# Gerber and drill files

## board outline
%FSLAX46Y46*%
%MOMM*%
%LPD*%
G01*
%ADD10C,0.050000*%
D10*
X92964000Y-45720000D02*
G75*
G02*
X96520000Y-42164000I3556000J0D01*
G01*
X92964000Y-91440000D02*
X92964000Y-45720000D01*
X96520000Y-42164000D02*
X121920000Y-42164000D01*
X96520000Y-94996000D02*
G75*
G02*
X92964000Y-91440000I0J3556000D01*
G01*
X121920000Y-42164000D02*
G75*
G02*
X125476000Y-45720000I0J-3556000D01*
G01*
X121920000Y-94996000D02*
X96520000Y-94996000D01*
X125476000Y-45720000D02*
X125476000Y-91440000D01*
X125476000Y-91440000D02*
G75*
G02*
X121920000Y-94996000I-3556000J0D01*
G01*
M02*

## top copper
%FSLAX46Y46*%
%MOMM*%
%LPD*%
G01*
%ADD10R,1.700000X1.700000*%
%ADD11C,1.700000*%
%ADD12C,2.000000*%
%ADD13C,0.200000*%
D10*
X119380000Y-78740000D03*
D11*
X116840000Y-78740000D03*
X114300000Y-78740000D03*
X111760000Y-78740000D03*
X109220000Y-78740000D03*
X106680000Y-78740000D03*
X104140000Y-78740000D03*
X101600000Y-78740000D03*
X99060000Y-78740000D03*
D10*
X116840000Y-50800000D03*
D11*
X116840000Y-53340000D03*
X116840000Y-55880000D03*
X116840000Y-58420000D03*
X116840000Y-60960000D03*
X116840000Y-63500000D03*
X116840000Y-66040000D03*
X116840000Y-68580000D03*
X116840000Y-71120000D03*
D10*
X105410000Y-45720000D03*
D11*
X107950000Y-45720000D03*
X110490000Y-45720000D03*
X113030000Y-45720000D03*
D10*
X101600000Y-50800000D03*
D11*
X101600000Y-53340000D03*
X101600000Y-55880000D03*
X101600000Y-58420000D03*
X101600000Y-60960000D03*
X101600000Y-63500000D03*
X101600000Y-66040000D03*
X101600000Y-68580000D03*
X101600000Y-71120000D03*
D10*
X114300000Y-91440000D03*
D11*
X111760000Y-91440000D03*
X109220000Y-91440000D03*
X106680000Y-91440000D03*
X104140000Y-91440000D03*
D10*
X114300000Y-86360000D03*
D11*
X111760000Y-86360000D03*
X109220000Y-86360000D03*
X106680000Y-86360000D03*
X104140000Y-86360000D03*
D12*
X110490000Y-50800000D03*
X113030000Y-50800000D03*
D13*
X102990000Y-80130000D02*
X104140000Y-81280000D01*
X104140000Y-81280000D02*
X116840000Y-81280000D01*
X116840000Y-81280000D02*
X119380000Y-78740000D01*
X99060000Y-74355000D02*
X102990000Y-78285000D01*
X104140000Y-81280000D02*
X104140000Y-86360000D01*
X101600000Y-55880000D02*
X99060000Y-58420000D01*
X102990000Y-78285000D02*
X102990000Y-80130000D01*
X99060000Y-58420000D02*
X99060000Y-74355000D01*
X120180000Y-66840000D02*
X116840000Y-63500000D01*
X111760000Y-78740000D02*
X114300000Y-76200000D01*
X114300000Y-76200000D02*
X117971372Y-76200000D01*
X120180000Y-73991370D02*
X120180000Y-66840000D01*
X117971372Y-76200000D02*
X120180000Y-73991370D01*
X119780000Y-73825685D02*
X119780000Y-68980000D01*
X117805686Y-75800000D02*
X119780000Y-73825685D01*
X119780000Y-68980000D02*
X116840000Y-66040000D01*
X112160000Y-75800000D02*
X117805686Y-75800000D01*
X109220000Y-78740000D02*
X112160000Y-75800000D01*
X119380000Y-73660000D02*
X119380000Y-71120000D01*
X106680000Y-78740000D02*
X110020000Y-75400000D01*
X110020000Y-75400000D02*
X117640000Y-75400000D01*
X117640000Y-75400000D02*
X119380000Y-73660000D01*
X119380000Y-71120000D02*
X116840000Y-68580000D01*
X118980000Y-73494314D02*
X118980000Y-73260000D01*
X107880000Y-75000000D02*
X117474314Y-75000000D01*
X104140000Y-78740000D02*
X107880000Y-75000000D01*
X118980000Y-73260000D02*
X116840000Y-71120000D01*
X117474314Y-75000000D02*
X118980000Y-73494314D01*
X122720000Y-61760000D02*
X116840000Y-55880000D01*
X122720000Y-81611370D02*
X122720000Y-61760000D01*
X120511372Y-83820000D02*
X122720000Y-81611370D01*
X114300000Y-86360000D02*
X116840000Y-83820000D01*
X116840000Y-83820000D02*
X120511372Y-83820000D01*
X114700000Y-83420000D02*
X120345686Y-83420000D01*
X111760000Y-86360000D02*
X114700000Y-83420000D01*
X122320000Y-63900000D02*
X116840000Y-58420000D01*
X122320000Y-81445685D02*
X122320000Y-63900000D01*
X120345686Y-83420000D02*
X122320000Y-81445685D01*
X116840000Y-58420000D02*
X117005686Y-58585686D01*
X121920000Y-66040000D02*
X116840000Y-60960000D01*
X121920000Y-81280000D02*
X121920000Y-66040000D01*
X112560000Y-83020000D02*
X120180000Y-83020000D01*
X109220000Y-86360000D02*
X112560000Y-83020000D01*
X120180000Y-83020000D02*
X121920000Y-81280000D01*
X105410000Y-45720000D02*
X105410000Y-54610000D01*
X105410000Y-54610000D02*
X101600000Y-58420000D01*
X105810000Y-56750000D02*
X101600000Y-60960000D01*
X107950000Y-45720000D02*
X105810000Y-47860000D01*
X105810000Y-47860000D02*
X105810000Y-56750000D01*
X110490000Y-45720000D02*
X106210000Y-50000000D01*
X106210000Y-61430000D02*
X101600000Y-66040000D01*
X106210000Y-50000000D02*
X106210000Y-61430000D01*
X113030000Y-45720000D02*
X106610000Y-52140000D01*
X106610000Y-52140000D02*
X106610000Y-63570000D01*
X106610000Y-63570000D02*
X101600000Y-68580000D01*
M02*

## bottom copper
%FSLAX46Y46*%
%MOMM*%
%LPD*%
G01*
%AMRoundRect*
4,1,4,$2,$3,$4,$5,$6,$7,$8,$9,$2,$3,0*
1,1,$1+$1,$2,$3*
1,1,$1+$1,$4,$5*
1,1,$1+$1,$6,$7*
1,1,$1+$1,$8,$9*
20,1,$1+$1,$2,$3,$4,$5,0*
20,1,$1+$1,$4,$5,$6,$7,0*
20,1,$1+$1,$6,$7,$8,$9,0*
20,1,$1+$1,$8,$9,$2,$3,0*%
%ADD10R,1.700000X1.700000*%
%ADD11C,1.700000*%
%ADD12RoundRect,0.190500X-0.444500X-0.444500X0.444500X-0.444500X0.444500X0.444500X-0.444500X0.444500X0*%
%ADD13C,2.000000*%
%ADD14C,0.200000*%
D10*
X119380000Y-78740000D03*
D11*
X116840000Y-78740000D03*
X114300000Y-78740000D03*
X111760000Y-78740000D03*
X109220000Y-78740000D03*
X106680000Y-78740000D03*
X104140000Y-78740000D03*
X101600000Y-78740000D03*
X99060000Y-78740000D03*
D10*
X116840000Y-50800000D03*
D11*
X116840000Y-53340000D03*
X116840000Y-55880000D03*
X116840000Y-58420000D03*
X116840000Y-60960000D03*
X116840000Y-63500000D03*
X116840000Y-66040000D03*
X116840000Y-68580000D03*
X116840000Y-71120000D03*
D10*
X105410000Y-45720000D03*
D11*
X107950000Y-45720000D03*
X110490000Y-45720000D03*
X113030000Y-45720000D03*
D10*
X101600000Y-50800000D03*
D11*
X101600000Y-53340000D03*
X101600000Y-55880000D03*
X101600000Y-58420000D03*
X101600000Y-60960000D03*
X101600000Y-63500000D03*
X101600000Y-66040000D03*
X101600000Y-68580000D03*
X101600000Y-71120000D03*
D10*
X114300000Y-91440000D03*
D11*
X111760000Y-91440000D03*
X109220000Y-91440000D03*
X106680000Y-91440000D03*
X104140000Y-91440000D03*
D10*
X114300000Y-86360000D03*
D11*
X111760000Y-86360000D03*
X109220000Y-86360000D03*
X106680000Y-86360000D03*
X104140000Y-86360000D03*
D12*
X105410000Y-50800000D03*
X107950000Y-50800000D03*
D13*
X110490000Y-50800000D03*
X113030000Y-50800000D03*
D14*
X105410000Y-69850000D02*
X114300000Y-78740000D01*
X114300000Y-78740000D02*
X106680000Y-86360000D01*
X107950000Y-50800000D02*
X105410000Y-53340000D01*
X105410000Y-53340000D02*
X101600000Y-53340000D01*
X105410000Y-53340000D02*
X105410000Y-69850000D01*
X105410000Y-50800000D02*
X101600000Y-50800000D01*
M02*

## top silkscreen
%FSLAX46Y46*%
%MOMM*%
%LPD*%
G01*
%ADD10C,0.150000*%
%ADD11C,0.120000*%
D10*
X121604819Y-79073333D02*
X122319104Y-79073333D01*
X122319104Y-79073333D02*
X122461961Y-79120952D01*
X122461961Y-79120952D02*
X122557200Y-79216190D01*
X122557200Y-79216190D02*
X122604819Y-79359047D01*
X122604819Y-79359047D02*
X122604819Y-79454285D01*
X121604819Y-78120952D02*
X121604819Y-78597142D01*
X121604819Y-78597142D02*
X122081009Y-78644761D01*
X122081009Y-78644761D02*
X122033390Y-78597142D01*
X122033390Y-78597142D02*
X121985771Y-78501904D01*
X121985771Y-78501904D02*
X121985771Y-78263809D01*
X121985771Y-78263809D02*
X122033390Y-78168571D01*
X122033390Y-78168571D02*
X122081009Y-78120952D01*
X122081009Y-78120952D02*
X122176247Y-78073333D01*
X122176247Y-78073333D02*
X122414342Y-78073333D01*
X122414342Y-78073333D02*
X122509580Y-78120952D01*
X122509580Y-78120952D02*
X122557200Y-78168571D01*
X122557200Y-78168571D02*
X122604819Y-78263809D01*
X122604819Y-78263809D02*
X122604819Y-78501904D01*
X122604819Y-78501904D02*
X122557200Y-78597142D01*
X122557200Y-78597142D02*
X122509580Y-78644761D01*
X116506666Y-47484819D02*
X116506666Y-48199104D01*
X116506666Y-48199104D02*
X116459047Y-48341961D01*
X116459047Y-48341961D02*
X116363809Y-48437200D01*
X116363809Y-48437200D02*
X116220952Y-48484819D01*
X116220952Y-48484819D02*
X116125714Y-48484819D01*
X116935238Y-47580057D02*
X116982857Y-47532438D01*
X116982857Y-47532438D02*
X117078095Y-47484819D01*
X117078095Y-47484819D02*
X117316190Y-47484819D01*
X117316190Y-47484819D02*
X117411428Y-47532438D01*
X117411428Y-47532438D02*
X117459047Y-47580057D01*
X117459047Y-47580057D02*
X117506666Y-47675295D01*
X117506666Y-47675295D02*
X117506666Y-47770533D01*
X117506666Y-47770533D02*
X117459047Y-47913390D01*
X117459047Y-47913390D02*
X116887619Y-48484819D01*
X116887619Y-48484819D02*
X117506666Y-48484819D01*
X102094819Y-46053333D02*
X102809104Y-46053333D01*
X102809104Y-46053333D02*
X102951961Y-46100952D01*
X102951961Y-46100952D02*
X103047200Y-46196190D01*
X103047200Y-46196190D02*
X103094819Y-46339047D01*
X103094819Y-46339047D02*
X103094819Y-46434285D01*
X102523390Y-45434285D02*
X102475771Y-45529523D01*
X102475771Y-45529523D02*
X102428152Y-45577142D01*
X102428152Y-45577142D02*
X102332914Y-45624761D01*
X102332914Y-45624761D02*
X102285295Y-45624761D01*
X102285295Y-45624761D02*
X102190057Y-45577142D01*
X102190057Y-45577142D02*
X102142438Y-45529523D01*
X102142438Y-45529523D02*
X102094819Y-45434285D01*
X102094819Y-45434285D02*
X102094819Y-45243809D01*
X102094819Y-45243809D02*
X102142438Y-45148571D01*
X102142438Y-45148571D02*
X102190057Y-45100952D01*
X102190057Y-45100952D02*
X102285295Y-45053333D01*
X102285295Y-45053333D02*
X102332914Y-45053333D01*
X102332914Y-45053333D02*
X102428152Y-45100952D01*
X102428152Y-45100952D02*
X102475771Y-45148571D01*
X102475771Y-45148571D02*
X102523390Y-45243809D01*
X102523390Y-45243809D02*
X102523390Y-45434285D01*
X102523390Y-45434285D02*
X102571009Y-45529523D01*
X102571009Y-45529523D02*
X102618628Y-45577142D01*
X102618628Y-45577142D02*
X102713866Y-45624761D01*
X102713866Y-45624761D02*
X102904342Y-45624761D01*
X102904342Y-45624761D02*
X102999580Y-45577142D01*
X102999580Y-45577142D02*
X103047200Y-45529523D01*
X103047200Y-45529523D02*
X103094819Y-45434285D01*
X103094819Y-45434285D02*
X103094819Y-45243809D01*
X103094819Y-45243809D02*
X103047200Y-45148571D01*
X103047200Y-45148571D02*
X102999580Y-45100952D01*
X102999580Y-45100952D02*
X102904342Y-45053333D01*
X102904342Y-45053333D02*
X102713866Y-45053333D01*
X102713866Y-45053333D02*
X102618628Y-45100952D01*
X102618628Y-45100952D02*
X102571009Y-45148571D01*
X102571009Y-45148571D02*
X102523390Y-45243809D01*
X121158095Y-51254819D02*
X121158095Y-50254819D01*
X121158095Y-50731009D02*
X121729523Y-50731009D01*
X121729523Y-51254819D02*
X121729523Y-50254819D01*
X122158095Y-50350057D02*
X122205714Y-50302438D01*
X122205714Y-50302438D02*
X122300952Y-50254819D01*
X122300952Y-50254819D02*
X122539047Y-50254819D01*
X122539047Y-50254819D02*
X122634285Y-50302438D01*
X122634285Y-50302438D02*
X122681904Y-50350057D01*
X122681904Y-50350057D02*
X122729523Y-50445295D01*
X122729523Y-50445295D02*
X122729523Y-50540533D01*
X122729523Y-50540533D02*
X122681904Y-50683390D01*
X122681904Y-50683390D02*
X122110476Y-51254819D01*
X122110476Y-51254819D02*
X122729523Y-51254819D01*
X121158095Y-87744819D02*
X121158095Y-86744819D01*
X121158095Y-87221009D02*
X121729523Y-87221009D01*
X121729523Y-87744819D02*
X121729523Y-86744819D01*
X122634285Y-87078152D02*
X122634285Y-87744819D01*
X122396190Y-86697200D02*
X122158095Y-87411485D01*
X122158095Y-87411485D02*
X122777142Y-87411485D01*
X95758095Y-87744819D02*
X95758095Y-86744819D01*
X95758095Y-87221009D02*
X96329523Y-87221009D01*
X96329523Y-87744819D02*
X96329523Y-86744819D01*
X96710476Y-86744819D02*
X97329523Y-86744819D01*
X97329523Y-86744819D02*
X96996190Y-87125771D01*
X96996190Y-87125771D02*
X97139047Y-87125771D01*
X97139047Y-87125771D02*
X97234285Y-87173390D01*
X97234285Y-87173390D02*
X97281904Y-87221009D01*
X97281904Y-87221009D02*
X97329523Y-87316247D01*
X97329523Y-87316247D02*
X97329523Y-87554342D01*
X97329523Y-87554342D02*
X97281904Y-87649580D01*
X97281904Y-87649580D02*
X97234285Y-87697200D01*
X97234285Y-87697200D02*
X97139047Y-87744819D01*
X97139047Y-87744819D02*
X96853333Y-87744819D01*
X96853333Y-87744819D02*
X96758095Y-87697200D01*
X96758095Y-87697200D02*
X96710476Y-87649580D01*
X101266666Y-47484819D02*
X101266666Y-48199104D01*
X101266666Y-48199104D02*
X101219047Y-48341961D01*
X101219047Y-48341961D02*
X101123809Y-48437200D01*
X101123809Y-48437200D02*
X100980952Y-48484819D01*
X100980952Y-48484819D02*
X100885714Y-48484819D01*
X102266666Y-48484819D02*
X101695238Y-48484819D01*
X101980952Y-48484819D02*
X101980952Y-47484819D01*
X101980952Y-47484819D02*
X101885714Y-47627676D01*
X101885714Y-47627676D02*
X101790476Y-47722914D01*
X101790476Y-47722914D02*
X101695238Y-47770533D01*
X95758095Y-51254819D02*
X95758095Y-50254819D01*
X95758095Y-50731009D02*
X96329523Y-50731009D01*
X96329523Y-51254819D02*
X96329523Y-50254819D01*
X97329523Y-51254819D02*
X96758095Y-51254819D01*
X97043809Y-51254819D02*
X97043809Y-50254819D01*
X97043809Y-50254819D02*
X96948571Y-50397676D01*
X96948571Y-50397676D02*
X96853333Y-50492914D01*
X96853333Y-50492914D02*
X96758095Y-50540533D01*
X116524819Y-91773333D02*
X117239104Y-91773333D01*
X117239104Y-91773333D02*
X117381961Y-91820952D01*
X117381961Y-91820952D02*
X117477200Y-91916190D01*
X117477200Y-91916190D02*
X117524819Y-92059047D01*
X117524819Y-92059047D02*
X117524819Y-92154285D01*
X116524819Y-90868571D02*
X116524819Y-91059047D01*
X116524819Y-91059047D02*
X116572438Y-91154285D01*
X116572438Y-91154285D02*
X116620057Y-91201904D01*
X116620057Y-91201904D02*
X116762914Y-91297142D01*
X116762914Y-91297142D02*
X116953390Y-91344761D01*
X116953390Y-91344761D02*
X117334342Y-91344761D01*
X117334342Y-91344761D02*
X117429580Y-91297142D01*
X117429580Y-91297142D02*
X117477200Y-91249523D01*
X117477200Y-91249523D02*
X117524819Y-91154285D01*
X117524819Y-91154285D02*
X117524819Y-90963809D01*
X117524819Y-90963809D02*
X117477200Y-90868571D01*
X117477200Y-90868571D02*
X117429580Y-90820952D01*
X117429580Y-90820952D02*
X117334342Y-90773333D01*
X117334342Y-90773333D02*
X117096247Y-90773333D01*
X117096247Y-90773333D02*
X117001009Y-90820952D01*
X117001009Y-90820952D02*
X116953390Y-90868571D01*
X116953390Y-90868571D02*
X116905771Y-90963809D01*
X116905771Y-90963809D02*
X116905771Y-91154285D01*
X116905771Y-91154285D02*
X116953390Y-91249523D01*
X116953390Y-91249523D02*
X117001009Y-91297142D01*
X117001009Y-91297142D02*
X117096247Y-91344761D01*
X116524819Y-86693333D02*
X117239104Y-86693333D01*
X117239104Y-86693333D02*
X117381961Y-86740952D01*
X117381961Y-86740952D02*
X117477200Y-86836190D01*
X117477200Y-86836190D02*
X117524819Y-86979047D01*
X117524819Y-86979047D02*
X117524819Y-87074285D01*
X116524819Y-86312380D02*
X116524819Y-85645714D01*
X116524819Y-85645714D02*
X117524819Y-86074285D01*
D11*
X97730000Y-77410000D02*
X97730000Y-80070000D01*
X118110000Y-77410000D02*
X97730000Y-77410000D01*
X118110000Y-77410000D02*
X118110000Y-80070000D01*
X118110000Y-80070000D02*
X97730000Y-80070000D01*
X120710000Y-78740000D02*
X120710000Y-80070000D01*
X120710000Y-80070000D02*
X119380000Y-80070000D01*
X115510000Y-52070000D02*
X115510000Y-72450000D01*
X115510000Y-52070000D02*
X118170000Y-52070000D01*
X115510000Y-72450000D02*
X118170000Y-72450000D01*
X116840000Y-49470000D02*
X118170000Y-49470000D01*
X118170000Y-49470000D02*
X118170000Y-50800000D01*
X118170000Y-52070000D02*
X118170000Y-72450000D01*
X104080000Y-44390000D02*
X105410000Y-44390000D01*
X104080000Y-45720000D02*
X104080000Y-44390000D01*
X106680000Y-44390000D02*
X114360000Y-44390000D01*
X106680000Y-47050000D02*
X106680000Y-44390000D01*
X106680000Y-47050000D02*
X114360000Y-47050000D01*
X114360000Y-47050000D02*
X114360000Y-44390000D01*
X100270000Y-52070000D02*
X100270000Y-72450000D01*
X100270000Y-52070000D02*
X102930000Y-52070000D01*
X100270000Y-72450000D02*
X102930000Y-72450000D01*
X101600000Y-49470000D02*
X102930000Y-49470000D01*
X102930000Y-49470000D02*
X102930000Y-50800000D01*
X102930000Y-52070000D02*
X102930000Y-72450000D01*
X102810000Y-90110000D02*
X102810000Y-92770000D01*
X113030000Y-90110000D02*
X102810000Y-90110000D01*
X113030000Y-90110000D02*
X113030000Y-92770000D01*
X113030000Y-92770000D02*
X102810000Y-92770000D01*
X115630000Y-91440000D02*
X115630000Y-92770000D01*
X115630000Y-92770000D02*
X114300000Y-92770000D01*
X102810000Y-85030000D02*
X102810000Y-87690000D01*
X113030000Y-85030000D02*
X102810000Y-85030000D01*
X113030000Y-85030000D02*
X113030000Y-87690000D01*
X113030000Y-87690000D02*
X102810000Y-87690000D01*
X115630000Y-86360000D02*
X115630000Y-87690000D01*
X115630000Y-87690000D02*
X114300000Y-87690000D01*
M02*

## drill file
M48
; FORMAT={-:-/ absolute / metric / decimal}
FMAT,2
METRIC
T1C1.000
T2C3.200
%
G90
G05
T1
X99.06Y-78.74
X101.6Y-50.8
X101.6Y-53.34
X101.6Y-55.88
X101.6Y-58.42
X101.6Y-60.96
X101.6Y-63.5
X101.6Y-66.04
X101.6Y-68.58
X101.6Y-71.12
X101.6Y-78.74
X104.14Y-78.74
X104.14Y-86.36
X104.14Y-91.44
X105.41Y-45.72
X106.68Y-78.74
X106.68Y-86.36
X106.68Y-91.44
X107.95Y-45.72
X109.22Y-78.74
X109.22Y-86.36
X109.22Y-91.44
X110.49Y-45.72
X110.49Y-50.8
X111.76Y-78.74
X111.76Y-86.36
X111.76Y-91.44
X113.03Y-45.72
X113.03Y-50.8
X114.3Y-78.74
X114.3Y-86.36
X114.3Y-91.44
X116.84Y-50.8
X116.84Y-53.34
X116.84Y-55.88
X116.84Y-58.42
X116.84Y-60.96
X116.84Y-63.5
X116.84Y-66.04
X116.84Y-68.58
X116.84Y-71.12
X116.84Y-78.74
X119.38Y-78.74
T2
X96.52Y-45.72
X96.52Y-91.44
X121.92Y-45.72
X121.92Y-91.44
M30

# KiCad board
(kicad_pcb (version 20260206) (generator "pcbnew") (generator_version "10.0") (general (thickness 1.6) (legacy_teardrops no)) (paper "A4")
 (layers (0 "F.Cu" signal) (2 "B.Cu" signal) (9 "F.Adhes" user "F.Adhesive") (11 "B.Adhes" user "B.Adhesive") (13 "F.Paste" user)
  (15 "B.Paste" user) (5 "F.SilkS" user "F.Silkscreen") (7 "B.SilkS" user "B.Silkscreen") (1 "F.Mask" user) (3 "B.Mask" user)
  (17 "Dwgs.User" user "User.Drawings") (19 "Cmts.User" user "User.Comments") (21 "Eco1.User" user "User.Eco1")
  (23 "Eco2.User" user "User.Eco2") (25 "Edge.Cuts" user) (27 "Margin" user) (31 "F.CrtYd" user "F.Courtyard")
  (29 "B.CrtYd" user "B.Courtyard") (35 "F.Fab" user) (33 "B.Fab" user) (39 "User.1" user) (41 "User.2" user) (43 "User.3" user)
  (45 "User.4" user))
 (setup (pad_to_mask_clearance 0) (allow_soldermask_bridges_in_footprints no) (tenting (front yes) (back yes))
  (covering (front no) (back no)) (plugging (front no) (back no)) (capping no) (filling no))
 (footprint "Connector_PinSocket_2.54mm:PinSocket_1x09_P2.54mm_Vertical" (layer "F.Cu") (at 119.38 78.74 -90)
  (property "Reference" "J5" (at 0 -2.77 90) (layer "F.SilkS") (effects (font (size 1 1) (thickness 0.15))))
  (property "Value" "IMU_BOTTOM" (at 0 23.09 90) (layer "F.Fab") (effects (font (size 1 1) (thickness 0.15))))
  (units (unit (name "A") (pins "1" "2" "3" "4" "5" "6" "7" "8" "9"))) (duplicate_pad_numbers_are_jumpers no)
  (fp_line (start -1.33 21.65) (end 1.33 21.65) (stroke (width 0.12) (type solid)) (layer "F.SilkS"))
  (fp_line (start -1.33 1.27) (end -1.33 21.65) (stroke (width 0.12) (type solid)) (layer "F.SilkS"))
  (fp_line (start -1.33 1.27) (end 1.33 1.27) (stroke (width 0.12) (type solid)) (layer "F.SilkS"))
  (fp_line (start 1.33 1.27) (end 1.33 21.65) (stroke (width 0.12) (type solid)) (layer "F.SilkS"))
  (fp_line (start 0 -1.33) (end 1.33 -1.33) (stroke (width 0.12) (type solid)) (layer "F.SilkS"))
  (fp_line (start 1.33 -1.33) (end 1.33 0) (stroke (width 0.12) (type solid)) (layer "F.SilkS"))
  (pad "1" thru_hole rect (at 0 0 270) (size 1.7 1.7) (drill 1) (layers "*.Cu" "*.Mask") (remove_unused_layers no) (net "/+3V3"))
  (pad "2" thru_hole circle (at 0 2.54 270) (size 1.7 1.7) (drill 1) (layers "*.Cu" "*.Mask") (remove_unused_layers no)
   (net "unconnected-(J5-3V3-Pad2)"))
  (pad "3" thru_hole circle (at 0 5.08 270) (size 1.7 1.7) (drill 1) (layers "*.Cu" "*.Mask") (remove_unused_layers no) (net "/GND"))
  (pad "4" thru_hole circle (at 0 7.62 270) (size 1.7 1.7) (drill 1) (layers "*.Cu" "*.Mask") (remove_unused_layers no) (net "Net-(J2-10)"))
  (pad "5" thru_hole circle (at 0 10.16 270) (size 1.7 1.7) (drill 1) (layers "*.Cu" "*.Mask") (remove_unused_layers no) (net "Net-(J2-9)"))
  (pad "6" thru_hole circle (at 0 12.7 270) (size 1.7 1.7) (drill 1) (layers "*.Cu" "*.Mask") (remove_unused_layers no) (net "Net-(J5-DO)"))
  (pad "7" thru_hole circle (at 0 15.24 270) (size 1.7 1.7) (drill 1) (layers "*.Cu" "*.Mask") (remove_unused_layers no) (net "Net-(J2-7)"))
  (pad "8" thru_hole circle (at 0 17.78 270) (size 1.7 1.7) (drill 1) (layers "*.Cu" "*.Mask") (remove_unused_layers no)
   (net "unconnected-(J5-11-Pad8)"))
  (pad "9" thru_hole circle (at 0 20.32 270) (size 1.7 1.7) (drill 1) (layers "*.Cu" "*.Mask") (remove_unused_layers no)
   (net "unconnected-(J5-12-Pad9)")))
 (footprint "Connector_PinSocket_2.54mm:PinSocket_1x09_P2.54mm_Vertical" (layer "F.Cu") (at 116.84 50.8)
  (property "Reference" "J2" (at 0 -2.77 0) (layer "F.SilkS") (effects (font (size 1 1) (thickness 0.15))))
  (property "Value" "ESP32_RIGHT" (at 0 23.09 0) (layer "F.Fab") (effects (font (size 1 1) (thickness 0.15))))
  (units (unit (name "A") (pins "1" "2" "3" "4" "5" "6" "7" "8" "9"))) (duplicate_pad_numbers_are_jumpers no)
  (fp_line (start -1.33 1.27) (end -1.33 21.65) (stroke (width 0.12) (type solid)) (layer "F.SilkS"))
  (fp_line (start -1.33 1.27) (end 1.33 1.27) (stroke (width 0.12) (type solid)) (layer "F.SilkS"))
  (fp_line (start -1.33 21.65) (end 1.33 21.65) (stroke (width 0.12) (type solid)) (layer "F.SilkS"))
  (fp_line (start 0 -1.33) (end 1.33 -1.33) (stroke (width 0.12) (type solid)) (layer "F.SilkS"))
  (fp_line (start 1.33 -1.33) (end 1.33 0) (stroke (width 0.12) (type solid)) (layer "F.SilkS"))
  (fp_line (start 1.33 1.27) (end 1.33 21.65) (stroke (width 0.12) (type solid)) (layer "F.SilkS"))
  (pad "1" thru_hole rect (at 0 0) (size 1.7 1.7) (drill 1) (layers "*.Cu" "*.Mask") (remove_unused_layers no)
   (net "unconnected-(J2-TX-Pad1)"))
  (pad "2" thru_hole circle (at 0 2.54) (size 1.7 1.7) (drill 1) (layers "*.Cu" "*.Mask") (remove_unused_layers no)
   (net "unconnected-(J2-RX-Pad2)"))
  (pad "3" thru_hole circle (at 0 5.08) (size 1.7 1.7) (drill 1) (layers "*.Cu" "*.Mask") (remove_unused_layers no) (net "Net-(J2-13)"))
  (pad "4" thru_hole circle (at 0 7.62) (size 1.7 1.7) (drill 1) (layers "*.Cu" "*.Mask") (remove_unused_layers no) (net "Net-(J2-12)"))
  (pad "5" thru_hole circle (at 0 10.16) (size 1.7 1.7) (drill 1) (layers "*.Cu" "*.Mask") (remove_unused_layers no) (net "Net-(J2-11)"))
  (pad "6" thru_hole circle (at 0 12.7) (size 1.7 1.7) (drill 1) (layers "*.Cu" "*.Mask") (remove_unused_layers no) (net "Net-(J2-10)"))
  (pad "7" thru_hole circle (at 0 15.24) (size 1.7 1.7) (drill 1) (layers "*.Cu" "*.Mask") (remove_unused_layers no) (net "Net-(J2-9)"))
  (pad "8" thru_hole circle (at 0 17.78) (size 1.7 1.7) (drill 1) (layers "*.Cu" "*.Mask") (remove_unused_layers no) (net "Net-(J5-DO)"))
  (pad "9" thru_hole circle (at 0 20.32) (size 1.7 1.7) (drill 1) (layers "*.Cu" "*.Mask") (remove_unused_layers no) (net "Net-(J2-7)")))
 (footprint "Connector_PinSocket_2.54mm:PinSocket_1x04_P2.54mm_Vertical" (layer "F.Cu") (at 105.41 45.72 90)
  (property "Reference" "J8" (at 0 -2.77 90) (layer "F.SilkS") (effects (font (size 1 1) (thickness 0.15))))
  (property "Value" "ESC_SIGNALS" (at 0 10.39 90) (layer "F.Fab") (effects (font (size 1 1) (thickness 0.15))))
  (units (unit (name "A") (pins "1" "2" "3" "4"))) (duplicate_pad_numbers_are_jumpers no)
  (fp_line (start 1.33 -1.33) (end 1.33 0) (stroke (width 0.12) (type solid)) (layer "F.SilkS"))
  (fp_line (start 0 -1.33) (end 1.33 -1.33) (stroke (width 0.12) (type solid)) (layer "F.SilkS"))
  (fp_line (start 1.33 1.27) (end 1.33 8.95) (stroke (width 0.12) (type solid)) (layer "F.SilkS"))
  (fp_line (start -1.33 1.27) (end 1.33 1.27) (stroke (width 0.12) (type solid)) (layer "F.SilkS"))
  (fp_line (start -1.33 1.27) (end -1.33 8.95) (stroke (width 0.12) (type solid)) (layer "F.SilkS"))
  (fp_line (start -1.33 8.95) (end 1.33 8.95) (stroke (width 0.12) (type solid)) (layer "F.SilkS"))
  (pad "1" thru_hole rect (at 0 0 90) (size 1.7 1.7) (drill 1) (layers "*.Cu" "*.Mask") (remove_unused_layers no) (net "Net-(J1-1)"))
  (pad "2" thru_hole circle (at 0 2.54 90) (size 1.7 1.7) (drill 1) (layers "*.Cu" "*.Mask") (remove_unused_layers no) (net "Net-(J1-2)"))
  (pad "3" thru_hole circle (at 0 5.08 90) (size 1.7 1.7) (drill 1) (layers "*.Cu" "*.Mask") (remove_unused_layers no) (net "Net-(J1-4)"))
  (pad "4" thru_hole circle (at 0 7.62 90) (size 1.7 1.7) (drill 1) (layers "*.Cu" "*.Mask") (remove_unused_layers no) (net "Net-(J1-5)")))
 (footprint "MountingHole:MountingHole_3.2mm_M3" (layer "F.Cu") (at 121.92 45.72)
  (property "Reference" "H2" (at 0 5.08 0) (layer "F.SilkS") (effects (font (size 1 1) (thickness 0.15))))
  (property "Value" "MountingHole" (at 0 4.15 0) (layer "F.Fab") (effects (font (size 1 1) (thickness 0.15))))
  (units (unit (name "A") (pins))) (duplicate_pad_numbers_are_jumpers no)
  (pad "" np_thru_hole circle (at 0 0) (size 3.2 3.2) (drill 3.2) (layers "*.Cu" "*.Mask")))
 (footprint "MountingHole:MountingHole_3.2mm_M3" (layer "F.Cu") (at 121.92 91.44)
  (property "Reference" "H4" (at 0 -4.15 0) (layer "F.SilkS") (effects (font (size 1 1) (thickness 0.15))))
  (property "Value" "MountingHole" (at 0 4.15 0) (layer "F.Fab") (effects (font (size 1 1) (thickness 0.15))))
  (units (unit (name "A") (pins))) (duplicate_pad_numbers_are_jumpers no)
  (pad "" np_thru_hole circle (at 0 0) (size 3.2 3.2) (drill 3.2) (layers "*.Cu" "*.Mask")))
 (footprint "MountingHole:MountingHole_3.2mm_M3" (layer "F.Cu") (at 96.52 91.44)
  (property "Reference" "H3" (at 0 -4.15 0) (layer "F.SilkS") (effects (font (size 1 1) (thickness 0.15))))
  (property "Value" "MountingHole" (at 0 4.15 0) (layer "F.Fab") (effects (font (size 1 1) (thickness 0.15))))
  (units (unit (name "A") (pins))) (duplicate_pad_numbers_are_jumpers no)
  (pad "" np_thru_hole circle (at 0 0) (size 3.2 3.2) (drill 3.2) (layers "*.Cu" "*.Mask")))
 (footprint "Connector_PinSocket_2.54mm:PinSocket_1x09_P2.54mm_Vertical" (layer "F.Cu") (at 101.6 50.8)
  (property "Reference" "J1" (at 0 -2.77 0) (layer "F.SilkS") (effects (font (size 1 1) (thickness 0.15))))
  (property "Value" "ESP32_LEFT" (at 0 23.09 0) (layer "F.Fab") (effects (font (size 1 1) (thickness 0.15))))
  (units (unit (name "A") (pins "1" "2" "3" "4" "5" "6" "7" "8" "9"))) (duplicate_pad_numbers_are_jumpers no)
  (fp_line (start -1.33 1.27) (end -1.33 21.65) (stroke (width 0.12) (type solid)) (layer "F.SilkS"))
  (fp_line (start -1.33 1.27) (end 1.33 1.27) (stroke (width 0.12) (type solid)) (layer "F.SilkS"))
  (fp_line (start -1.33 21.65) (end 1.33 21.65) (stroke (width 0.12) (type solid)) (layer "F.SilkS"))
  (fp_line (start 0 -1.33) (end 1.33 -1.33) (stroke (width 0.12) (type solid)) (layer "F.SilkS"))
  (fp_line (start 1.33 -1.33) (end 1.33 0) (stroke (width 0.12) (type solid)) (layer "F.SilkS"))
  (fp_line (start 1.33 1.27) (end 1.33 21.65) (stroke (width 0.12) (type solid)) (layer "F.SilkS"))
  (pad "1" thru_hole rect (at 0 0) (size 1.7 1.7) (drill 1) (layers "*.Cu" "*.Mask") (remove_unused_layers no) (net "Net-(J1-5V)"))
  (pad "2" thru_hole circle (at 0 2.54) (size 1.7 1.7) (drill 1) (layers "*.Cu" "*.Mask") (remove_unused_layers no) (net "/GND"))
  (pad "3" thru_hole circle (at 0 5.08) (size 1.7 1.7) (drill 1) (layers "*.Cu" "*.Mask") (remove_unused_layers no) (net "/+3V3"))
  (pad "4" thru_hole circle (at 0 7.62) (size 1.7 1.7) (drill 1) (layers "*.Cu" "*.Mask") (remove_unused_layers no) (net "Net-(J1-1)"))
  (pad "5" thru_hole circle (at 0 10.16) (size 1.7 1.7) (drill 1) (layers "*.Cu" "*.Mask") (remove_unused_layers no) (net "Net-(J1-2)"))
  (pad "6" thru_hole circle (at 0 12.7) (size 1.7 1.7) (drill 1) (layers "*.Cu" "*.Mask") (remove_unused_layers no)
   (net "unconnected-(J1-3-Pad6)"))
  (pad "7" thru_hole circle (at 0 15.24) (size 1.7 1.7) (drill 1) (layers "*.Cu" "*.Mask") (remove_unused_layers no) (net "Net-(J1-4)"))
  (pad "8" thru_hole circle (at 0 17.78) (size 1.7 1.7) (drill 1) (layers "*.Cu" "*.Mask") (remove_unused_layers no) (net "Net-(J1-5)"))
  (pad "9" thru_hole circle (at 0 20.32) (size 1.7 1.7) (drill 1) (layers "*.Cu" "*.Mask") (remove_unused_layers no)
   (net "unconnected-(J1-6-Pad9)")))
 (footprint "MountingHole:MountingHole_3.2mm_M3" (layer "F.Cu") (at 96.52 45.72)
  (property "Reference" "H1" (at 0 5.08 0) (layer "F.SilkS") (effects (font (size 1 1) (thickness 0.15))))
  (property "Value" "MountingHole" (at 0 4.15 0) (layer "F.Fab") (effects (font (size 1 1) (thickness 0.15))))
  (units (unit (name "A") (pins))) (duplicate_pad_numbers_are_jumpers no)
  (pad "" np_thru_hole circle (at 0 0) (size 3.2 3.2) (drill 3.2) (layers "*.Cu" "*.Mask")))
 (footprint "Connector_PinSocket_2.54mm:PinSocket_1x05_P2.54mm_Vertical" (layer "F.Cu") (at 114.3 91.44 -90)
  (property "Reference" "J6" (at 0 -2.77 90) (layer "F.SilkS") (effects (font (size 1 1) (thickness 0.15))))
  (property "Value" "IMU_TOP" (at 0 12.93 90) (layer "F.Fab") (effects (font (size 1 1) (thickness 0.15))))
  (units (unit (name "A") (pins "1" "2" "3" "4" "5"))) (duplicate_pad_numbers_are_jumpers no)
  (fp_line (start -1.33 11.49) (end 1.33 11.49) (stroke (width 0.12) (type solid)) (layer "F.SilkS"))
  (fp_line (start -1.33 1.27) (end -1.33 11.49) (stroke (width 0.12) (type solid)) (layer "F.SilkS"))
  (fp_line (start -1.33 1.27) (end 1.33 1.27) (stroke (width 0.12) (type solid)) (layer "F.SilkS"))
  (fp_line (start 1.33 1.27) (end 1.33 11.49) (stroke (width 0.12) (type solid)) (layer "F.SilkS"))
  (fp_line (start 0 -1.33) (end 1.33 -1.33) (stroke (width 0.12) (type solid)) (layer "F.SilkS"))
  (fp_line (start 1.33 -1.33) (end 1.33 0) (stroke (width 0.12) (type solid)) (layer "F.SilkS"))
  (pad "1" thru_hole rect (at 0 0 270) (size 1.7 1.7) (drill 1) (layers "*.Cu" "*.Mask") (remove_unused_layers no)
   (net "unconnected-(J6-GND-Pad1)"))
  (pad "2" thru_hole circle (at 0 2.54 270) (size 1.7 1.7) (drill 1) (layers "*.Cu" "*.Mask") (remove_unused_layers no)
   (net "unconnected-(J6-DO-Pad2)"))
  (pad "3" thru_hole circle (at 0 5.08 270) (size 1.7 1.7) (drill 1) (layers "*.Cu" "*.Mask") (remove_unused_layers no)
   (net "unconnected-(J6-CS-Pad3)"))
  (pad "4" thru_hole circle (at 0 7.62 270) (size 1.7 1.7) (drill 1) (layers "*.Cu" "*.Mask") (remove_unused_layers no)
   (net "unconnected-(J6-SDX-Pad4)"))
  (pad "5" thru_hole circle (at 0 10.16 270) (size 1.7 1.7) (drill 1) (layers "*.Cu" "*.Mask") (remove_unused_layers no)
   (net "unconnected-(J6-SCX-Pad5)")))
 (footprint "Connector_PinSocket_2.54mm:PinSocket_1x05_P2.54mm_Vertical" (layer "F.Cu") (at 114.3 86.36 -90)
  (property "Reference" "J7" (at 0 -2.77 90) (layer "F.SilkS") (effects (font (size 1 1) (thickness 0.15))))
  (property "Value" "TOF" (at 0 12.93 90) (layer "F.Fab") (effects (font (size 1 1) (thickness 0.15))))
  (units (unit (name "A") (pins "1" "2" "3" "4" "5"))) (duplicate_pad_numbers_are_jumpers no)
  (fp_line (start -1.33 11.49) (end 1.33 11.49) (stroke (width 0.12) (type solid)) (layer "F.SilkS"))
  (fp_line (start -1.33 1.27) (end -1.33 11.49) (stroke (width 0.12) (type solid)) (layer "F.SilkS"))
  (fp_line (start -1.33 1.27) (end 1.33 1.27) (stroke (width 0.12) (type solid)) (layer "F.SilkS"))
  (fp_line (start 1.33 1.27) (end 1.33 11.49) (stroke (width 0.12) (type solid)) (layer "F.SilkS"))
  (fp_line (start 0 -1.33) (end 1.33 -1.33) (stroke (width 0.12) (type solid)) (layer "F.SilkS"))
  (fp_line (start 1.33 -1.33) (end 1.33 0) (stroke (width 0.12) (type solid)) (layer "F.SilkS"))
  (pad "1" thru_hole rect (at 0 0 270) (size 1.7 1.7) (drill 1) (layers "*.Cu" "*.Mask") (remove_unused_layers no) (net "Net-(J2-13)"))
  (pad "2" thru_hole circle (at 0 2.54 270) (size 1.7 1.7) (drill 1) (layers "*.Cu" "*.Mask") (remove_unused_layers no) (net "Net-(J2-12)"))
  (pad "3" thru_hole circle (at 0 5.08 270) (size 1.7 1.7) (drill 1) (layers "*.Cu" "*.Mask") (remove_unused_layers no) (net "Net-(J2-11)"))
  (pad "4" thru_hole circle (at 0 7.62 270) (size 1.7 1.7) (drill 1) (layers "*.Cu" "*.Mask") (remove_unused_layers no) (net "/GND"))
  (pad "5" thru_hole circle (at 0 10.16 270) (size 1.7 1.7) (drill 1) (layers "*.Cu" "*.Mask") (remove_unused_layers no) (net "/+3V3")))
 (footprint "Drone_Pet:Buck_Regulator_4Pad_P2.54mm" (layer "B.Cu") (at 105.41 50.8)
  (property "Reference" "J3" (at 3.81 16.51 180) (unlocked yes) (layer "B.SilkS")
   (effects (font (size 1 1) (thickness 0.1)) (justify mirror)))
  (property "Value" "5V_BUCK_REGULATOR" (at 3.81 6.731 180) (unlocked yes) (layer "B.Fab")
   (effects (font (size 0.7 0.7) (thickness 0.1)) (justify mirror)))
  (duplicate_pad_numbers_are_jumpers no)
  (pad "1" smd roundrect (at 0 0) (size 1.27 1.27) (layers "B.Cu" "B.Mask" "B.Paste") (roundrect_rratio 0.15) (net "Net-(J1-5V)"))
  (pad "2" smd roundrect (at 2.54 0) (size 1.27 1.27) (layers "B.Cu" "B.Mask" "B.Paste") (roundrect_rratio 0.15) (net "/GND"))
  (pad "3" thru_hole circle (at 5.08 0) (size 2 2) (drill 1) (layers "*.Cu" "*.Mask") (remove_unused_layers no) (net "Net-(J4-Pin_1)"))
  (pad "4" thru_hole circle (at 7.62 0) (size 2 2) (drill 1) (layers "*.Cu" "*.Mask") (remove_unused_layers no) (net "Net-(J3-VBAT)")))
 (gr_arc (start 92.964 45.72) (mid 94.005528 43.205528) (end 96.52 42.164) (stroke (width 0.05) (type default)) (layer "Edge.Cuts"))
 (gr_line (start 92.964 91.44) (end 92.964 45.72) (stroke (width 0.05) (type default)) (layer "Edge.Cuts"))
 (gr_line (start 96.52 42.164) (end 121.92 42.164) (stroke (width 0.05) (type default)) (layer "Edge.Cuts"))
 (gr_arc (start 96.52 94.996) (mid 94.005528 93.954472) (end 92.964 91.44) (stroke (width 0.05) (type default)) (layer "Edge.Cuts"))
 (gr_arc (start 121.92 42.164) (mid 124.434472 43.205528) (end 125.476 45.72) (stroke (width 0.05) (type default)) (layer "Edge.Cuts"))
 (gr_line (start 121.92 94.996) (end 96.52 94.996) (stroke (width 0.05) (type default)) (layer "Edge.Cuts"))
 (gr_line (start 125.476 45.72) (end 125.476 91.44) (stroke (width 0.05) (type default)) (layer "Edge.Cuts"))
 (gr_arc (start 125.476 91.44) (mid 124.434472 93.954472) (end 121.92 94.996) (stroke (width 0.05) (type default)) (layer "Edge.Cuts"))
 (segment (start 102.99 80.13) (end 104.14 81.28) (width 0.2) (layer "F.Cu") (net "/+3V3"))
 (segment (start 104.14 81.28) (end 116.84 81.28) (width 0.2) (layer "F.Cu") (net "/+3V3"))
 (segment (start 116.84 81.28) (end 119.38 78.74) (width 0.2) (layer "F.Cu") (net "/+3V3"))
 (segment (start 99.06 74.355) (end 102.99 78.285) (width 0.2) (layer "F.Cu") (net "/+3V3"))
 (segment (start 104.14 81.28) (end 104.14 86.36) (width 0.2) (layer "F.Cu") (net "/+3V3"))
 (segment (start 101.6 55.88) (end 99.06 58.42) (width 0.2) (layer "F.Cu") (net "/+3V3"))
 (segment (start 102.99 78.285) (end 102.99 80.13) (width 0.2) (layer "F.Cu") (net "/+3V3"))
 (segment (start 99.06 58.42) (end 99.06 74.355) (width 0.2) (layer "F.Cu") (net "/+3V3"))
 (segment (start 105.41 69.85) (end 114.3 78.74) (width 0.2) (layer "B.Cu") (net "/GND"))
 (segment (start 114.3 78.74) (end 106.68 86.36) (width 0.2) (layer "B.Cu") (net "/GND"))
 (segment (start 107.95 50.8) (end 105.41 53.34) (width 0.2) (layer "B.Cu") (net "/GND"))
 (segment (start 105.41 53.34) (end 101.6 53.34) (width 0.2) (layer "B.Cu") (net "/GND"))
 (segment (start 105.41 53.34) (end 105.41 69.85) (width 0.2) (layer "B.Cu") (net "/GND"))
 (segment (start 120.18 66.84) (end 116.84 63.5) (width 0.2) (layer "F.Cu") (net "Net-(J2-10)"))
 (segment (start 111.76 78.74) (end 114.3 76.2) (width 0.2) (layer "F.Cu") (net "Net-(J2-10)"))
 (segment (start 114.3 76.2) (end 117.971372 76.2) (width 0.2) (layer "F.Cu") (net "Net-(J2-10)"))
 (segment (start 120.18 73.99137) (end 120.18 66.84) (width 0.2) (layer "F.Cu") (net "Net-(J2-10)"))
 (segment (start 117.971372 76.2) (end 120.18 73.99137) (width 0.2) (layer "F.Cu") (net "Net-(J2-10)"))
 (segment (start 119.78 73.825685) (end 119.78 68.98) (width 0.2) (layer "F.Cu") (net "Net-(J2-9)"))
 (segment (start 117.805686 75.8) (end 119.78 73.825685) (width 0.2) (layer "F.Cu") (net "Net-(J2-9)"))
 (segment (start 119.78 68.98) (end 116.84 66.04) (width 0.2) (layer "F.Cu") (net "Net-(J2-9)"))
 (segment (start 112.16 75.8) (end 117.805686 75.8) (width 0.2) (layer "F.Cu") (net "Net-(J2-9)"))
 (segment (start 109.22 78.74) (end 112.16 75.8) (width 0.2) (layer "F.Cu") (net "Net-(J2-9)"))
 (segment (start 119.38 73.66) (end 119.38 71.12) (width 0.2) (layer "F.Cu") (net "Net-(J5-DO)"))
 (segment (start 106.68 78.74) (end 110.02 75.4) (width 0.2) (layer "F.Cu") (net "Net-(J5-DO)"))
 (segment (start 110.02 75.4) (end 117.64 75.4) (width 0.2) (layer "F.Cu") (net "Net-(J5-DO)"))
 (segment (start 117.64 75.4) (end 119.38 73.66) (width 0.2) (layer "F.Cu") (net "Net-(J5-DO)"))
 (segment (start 119.38 71.12) (end 116.84 68.58) (width 0.2) (layer "F.Cu") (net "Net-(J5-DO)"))
 (segment (start 118.98 73.494314) (end 118.98 73.26) (width 0.2) (layer "F.Cu") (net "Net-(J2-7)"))
 (segment (start 107.88 75) (end 117.474314 75) (width 0.2) (layer "F.Cu") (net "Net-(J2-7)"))
 (segment (start 104.14 78.74) (end 107.88 75) (width 0.2) (layer "F.Cu") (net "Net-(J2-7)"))
 (segment (start 118.98 73.26) (end 116.84 71.12) (width 0.2) (layer "F.Cu") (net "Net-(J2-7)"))
 (segment (start 117.474314 75) (end 118.98 73.494314) (width 0.2) (layer "F.Cu") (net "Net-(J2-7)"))
 (segment (start 122.72 61.76) (end 116.84 55.88) (width 0.2) (layer "F.Cu") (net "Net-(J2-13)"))
 (segment (start 122.72 81.61137) (end 122.72 61.76) (width 0.2) (layer "F.Cu") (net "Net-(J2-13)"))
 (segment (start 120.511372 83.82) (end 122.72 81.61137) (width 0.2) (layer "F.Cu") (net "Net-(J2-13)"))
 (segment (start 114.3 86.36) (end 116.84 83.82) (width 0.2) (layer "F.Cu") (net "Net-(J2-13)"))
 (segment (start 116.84 83.82) (end 120.511372 83.82) (width 0.2) (layer "F.Cu") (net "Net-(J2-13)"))
 (segment (start 114.7 83.42) (end 120.345686 83.42) (width 0.2) (layer "F.Cu") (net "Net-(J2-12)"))
 (segment (start 111.76 86.36) (end 114.7 83.42) (width 0.2) (layer "F.Cu") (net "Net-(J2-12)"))
 (segment (start 122.32 63.9) (end 116.84 58.42) (width 0.2) (layer "F.Cu") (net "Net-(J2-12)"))
 (segment (start 122.32 81.445685) (end 122.32 63.9) (width 0.2) (layer "F.Cu") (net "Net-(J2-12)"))
 (segment (start 120.345686 83.42) (end 122.32 81.445685) (width 0.2) (layer "F.Cu") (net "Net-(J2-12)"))
 (segment (start 116.84 58.42) (end 117.005686 58.585686) (width 0.2) (layer "F.Cu") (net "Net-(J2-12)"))
 (segment (start 121.92 66.04) (end 116.84 60.96) (width 0.2) (layer "F.Cu") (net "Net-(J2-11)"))
 (segment (start 121.92 81.28) (end 121.92 66.04) (width 0.2) (layer "F.Cu") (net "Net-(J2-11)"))
 (segment (start 112.56 83.02) (end 120.18 83.02) (width 0.2) (layer "F.Cu") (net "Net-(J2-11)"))
 (segment (start 109.22 86.36) (end 112.56 83.02) (width 0.2) (layer "F.Cu") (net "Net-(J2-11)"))
 (segment (start 120.18 83.02) (end 121.92 81.28) (width 0.2) (layer "F.Cu") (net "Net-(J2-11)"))
 (segment (start 105.41 45.72) (end 105.41 54.61) (width 0.2) (layer "F.Cu") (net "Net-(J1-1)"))
 (segment (start 105.41 54.61) (end 101.6 58.42) (width 0.2) (layer "F.Cu") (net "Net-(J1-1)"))
 (segment (start 105.81 56.75) (end 101.6 60.96) (width 0.2) (layer "F.Cu") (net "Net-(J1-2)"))
 (segment (start 107.95 45.72) (end 105.81 47.86) (width 0.2) (layer "F.Cu") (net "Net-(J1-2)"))
 (segment (start 105.81 47.86) (end 105.81 56.75) (width 0.2) (layer "F.Cu") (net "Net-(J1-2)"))
 (segment (start 110.49 45.72) (end 106.21 50) (width 0.2) (layer "F.Cu") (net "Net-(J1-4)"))
 (segment (start 106.21 61.43) (end 101.6 66.04) (width 0.2) (layer "F.Cu") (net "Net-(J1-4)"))
 (segment (start 106.21 50) (end 106.21 61.43) (width 0.2) (layer "F.Cu") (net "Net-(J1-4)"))
 (segment (start 113.03 45.72) (end 106.61 52.14) (width 0.2) (layer "F.Cu") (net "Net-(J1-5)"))
 (segment (start 106.61 52.14) (end 106.61 63.57) (width 0.2) (layer "F.Cu") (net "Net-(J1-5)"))
 (segment (start 106.61 63.57) (end 101.6 68.58) (width 0.2) (layer "F.Cu") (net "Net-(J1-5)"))
 (segment (start 105.41 50.8) (end 101.6 50.8) (width 0.2) (layer "B.Cu") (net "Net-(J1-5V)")))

